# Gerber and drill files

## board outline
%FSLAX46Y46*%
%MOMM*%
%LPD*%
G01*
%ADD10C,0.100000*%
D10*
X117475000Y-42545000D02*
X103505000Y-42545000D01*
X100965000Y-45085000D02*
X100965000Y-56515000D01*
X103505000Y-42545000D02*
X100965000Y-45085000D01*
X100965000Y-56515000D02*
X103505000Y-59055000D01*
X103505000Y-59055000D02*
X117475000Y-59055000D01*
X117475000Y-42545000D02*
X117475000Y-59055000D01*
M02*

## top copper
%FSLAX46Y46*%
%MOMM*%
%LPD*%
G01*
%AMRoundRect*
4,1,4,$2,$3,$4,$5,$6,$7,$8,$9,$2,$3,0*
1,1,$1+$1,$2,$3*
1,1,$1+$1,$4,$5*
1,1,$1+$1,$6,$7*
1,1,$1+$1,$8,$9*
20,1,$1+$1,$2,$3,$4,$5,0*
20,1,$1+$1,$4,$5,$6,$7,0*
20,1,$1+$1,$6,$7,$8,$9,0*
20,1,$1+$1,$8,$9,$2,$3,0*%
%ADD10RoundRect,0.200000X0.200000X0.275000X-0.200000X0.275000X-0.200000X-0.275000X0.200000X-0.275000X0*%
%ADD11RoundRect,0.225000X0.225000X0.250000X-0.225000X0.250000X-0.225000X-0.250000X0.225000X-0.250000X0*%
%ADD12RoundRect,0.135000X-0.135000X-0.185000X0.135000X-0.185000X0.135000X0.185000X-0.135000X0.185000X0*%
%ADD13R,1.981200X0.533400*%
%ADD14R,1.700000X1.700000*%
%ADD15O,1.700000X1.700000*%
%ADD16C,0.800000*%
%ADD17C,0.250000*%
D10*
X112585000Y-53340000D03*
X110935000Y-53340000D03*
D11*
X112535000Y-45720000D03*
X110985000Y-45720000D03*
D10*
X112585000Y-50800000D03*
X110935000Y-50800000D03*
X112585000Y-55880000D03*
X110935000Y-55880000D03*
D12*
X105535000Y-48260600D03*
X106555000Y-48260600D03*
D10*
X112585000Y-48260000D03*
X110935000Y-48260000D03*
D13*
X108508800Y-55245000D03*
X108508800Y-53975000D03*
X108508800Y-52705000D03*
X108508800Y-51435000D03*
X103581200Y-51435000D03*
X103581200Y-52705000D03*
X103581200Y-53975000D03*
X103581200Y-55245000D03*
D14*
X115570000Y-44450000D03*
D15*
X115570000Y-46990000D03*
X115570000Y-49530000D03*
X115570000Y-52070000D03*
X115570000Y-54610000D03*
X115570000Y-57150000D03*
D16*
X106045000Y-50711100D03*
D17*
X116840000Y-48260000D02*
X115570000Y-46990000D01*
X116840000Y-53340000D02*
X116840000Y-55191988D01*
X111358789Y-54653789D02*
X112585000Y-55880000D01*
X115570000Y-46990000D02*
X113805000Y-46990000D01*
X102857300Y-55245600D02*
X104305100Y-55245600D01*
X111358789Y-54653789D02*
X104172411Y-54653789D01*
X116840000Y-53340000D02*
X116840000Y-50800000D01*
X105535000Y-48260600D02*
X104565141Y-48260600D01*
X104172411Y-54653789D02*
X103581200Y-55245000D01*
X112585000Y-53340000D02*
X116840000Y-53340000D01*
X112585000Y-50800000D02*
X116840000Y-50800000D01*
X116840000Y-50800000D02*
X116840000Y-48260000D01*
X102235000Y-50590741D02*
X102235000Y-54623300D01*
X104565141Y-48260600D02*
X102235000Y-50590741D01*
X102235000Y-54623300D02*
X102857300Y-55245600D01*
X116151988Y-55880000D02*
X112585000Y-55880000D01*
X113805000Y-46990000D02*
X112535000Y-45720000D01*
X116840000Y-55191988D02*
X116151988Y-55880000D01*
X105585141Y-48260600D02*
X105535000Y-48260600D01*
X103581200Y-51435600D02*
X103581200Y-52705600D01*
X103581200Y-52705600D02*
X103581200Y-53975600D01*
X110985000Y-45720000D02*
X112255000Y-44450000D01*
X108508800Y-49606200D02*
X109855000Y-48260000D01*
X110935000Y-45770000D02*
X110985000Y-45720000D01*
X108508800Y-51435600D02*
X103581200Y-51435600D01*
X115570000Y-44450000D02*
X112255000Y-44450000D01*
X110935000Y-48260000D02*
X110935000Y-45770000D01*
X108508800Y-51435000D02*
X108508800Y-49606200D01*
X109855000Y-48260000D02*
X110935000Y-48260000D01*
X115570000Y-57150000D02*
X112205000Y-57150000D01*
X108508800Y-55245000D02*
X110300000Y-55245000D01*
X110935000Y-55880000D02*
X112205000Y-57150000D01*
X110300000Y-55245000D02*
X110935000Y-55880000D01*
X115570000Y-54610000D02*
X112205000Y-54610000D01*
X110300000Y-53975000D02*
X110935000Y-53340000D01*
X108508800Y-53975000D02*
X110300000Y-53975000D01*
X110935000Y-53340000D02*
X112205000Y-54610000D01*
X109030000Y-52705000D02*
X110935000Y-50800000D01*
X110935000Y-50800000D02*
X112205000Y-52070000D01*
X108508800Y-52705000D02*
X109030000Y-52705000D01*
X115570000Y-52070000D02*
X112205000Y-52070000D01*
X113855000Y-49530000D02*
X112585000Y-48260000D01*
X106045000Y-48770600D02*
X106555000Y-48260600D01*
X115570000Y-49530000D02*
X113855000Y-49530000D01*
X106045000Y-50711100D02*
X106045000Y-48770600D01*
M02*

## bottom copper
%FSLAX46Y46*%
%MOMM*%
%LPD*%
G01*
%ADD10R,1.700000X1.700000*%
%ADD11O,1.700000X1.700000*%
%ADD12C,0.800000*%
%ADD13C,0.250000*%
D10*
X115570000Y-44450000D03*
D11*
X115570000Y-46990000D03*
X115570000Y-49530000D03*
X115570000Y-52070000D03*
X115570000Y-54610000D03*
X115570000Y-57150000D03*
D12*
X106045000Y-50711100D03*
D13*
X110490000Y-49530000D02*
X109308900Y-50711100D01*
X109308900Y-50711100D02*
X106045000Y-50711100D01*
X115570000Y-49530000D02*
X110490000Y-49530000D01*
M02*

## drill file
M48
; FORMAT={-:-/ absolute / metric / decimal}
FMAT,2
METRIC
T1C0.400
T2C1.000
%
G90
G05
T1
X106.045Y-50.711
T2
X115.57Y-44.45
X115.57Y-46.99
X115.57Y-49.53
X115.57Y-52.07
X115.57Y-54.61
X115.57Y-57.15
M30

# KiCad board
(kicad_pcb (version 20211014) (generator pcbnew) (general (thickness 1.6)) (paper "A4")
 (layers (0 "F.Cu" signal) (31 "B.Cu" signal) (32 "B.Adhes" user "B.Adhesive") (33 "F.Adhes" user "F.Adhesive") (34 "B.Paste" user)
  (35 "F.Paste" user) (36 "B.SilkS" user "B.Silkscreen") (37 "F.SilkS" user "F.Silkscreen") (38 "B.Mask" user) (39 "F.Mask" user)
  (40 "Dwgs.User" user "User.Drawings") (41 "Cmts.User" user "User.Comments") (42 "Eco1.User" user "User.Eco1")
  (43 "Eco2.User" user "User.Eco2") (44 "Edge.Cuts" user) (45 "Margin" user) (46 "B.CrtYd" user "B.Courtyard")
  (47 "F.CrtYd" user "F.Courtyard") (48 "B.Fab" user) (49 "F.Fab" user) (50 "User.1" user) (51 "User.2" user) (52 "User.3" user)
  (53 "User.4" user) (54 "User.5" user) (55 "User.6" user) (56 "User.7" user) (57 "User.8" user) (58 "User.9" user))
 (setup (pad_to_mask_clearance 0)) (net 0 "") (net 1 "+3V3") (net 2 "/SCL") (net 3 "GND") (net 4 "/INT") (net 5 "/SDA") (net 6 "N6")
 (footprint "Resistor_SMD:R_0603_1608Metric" (layer "F.Cu") (at 111.76 53.34 180)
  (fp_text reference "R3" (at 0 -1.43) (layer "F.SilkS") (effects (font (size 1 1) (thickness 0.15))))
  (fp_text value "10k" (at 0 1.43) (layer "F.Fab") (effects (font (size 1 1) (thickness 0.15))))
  (pad "1" smd roundrect (at -0.825 0 180) (size 0.8 0.95) (layers "F.Cu" "F.Paste" "F.Mask") (roundrect_rratio 0.25) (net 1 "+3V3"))
  (pad "2" smd roundrect (at 0.825 0 180) (size 0.8 0.95) (layers "F.Cu" "F.Paste" "F.Mask") (roundrect_rratio 0.25) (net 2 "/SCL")))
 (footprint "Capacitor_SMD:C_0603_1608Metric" (layer "F.Cu") (at 111.76 45.72 180)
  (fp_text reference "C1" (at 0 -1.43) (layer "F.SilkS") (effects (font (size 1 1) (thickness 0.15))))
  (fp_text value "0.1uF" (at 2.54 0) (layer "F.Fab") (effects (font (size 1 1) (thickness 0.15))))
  (pad "1" smd roundrect (at -0.775 0 180) (size 0.9 0.95) (layers "F.Cu" "F.Paste" "F.Mask") (roundrect_rratio 0.25) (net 1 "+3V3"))
  (pad "2" smd roundrect (at 0.775 0 180) (size 0.9 0.95) (layers "F.Cu" "F.Paste" "F.Mask") (roundrect_rratio 0.25) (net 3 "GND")))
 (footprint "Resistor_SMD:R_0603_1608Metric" (layer "F.Cu") (at 111.76 50.8 180)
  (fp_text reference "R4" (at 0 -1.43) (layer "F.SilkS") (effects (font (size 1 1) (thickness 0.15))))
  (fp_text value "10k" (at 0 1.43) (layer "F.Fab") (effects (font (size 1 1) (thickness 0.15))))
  (pad "1" smd roundrect (at -0.825 0 180) (size 0.8 0.95) (layers "F.Cu" "F.Paste" "F.Mask") (roundrect_rratio 0.25) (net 1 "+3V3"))
  (pad "2" smd roundrect (at 0.825 0 180) (size 0.8 0.95) (layers "F.Cu" "F.Paste" "F.Mask") (roundrect_rratio 0.25) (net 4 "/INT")))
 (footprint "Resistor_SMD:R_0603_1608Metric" (layer "F.Cu") (at 111.76 55.88 180)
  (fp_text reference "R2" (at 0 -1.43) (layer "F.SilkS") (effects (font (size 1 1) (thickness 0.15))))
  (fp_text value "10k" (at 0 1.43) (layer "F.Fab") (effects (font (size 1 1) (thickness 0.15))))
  (pad "1" smd roundrect (at -0.825 0 180) (size 0.8 0.95) (layers "F.Cu" "F.Paste" "F.Mask") (roundrect_rratio 0.25) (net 1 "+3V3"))
  (pad "2" smd roundrect (at 0.825 0 180) (size 0.8 0.95) (layers "F.Cu" "F.Paste" "F.Mask") (roundrect_rratio 0.25) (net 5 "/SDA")))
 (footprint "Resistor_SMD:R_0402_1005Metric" (layer "F.Cu") (at 106.045 48.2606)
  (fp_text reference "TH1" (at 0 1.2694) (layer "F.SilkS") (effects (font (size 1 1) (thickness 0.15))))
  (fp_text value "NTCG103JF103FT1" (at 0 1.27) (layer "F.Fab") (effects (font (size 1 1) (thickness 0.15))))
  (pad "1" smd roundrect (at -0.51 0) (size 0.54 0.64) (layers "F.Cu" "F.Paste" "F.Mask") (roundrect_rratio 0.25) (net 1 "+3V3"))
  (pad "2" smd roundrect (at 0.51 0) (size 0.54 0.64) (layers "F.Cu" "F.Paste" "F.Mask") (roundrect_rratio 0.25) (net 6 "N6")))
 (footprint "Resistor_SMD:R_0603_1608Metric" (layer "F.Cu") (at 111.76 48.26 180)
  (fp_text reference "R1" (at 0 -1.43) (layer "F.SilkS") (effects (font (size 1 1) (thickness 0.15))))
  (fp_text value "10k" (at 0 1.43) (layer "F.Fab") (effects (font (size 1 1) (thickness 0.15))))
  (pad "1" smd roundrect (at -0.825 0 180) (size 0.8 0.95) (layers "F.Cu" "F.Paste" "F.Mask") (roundrect_rratio 0.25) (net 6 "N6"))
  (pad "2" smd roundrect (at 0.825 0 180) (size 0.8 0.95) (layers "F.Cu" "F.Paste" "F.Mask") (roundrect_rratio 0.25) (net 3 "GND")))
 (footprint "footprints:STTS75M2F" (layer "F.Cu") (at 106.045 53.34 180)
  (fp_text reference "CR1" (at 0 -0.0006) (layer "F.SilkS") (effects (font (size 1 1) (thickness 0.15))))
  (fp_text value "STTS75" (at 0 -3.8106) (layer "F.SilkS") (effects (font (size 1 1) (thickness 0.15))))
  (pad "1" smd rect locked (at -2.4638 -1.905 180) (size 1.9812 0.5334) (layers "F.Cu" "F.Paste" "F.Mask") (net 5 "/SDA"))
  (pad "2" smd rect locked (at -2.4638 -0.635 180) (size 1.9812 0.5334) (layers "F.Cu" "F.Paste" "F.Mask") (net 2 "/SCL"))
  (pad "3" smd rect locked (at -2.4638 0.635 180) (size 1.9812 0.5334) (layers "F.Cu" "F.Paste" "F.Mask") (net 4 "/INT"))
  (pad "4" smd rect locked (at -2.4638 1.905 180) (size 1.9812 0.5334) (layers "F.Cu" "F.Paste" "F.Mask") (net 3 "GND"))
  (pad "5" smd rect locked (at 2.4638 1.905 180) (size 1.9812 0.5334) (layers "F.Cu" "F.Paste" "F.Mask") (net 3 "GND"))
  (pad "6" smd rect locked (at 2.4638 0.635 180) (size 1.9812 0.5334) (layers "F.Cu" "F.Paste" "F.Mask") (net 3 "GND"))
  (pad "7" smd rect locked (at 2.4638 -0.635 180) (size 1.9812 0.5334) (layers "F.Cu" "F.Paste" "F.Mask") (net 3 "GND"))
  (pad "8" smd rect locked (at 2.4638 -1.905 180) (size 1.9812 0.5334) (layers "F.Cu" "F.Paste" "F.Mask") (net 1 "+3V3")))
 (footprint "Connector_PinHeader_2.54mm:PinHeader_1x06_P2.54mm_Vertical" (layer "F.Cu") (at 115.57 44.45)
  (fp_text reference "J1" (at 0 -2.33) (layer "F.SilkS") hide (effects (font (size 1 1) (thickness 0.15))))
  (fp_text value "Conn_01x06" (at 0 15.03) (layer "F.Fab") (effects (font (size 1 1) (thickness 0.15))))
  (pad "1" thru_hole rect (at 0 0) (size 1.7 1.7) (drill 1) (layers *.Cu *.Mask) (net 3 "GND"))
  (pad "2" thru_hole oval (at 0 2.54) (size 1.7 1.7) (drill 1) (layers *.Cu *.Mask) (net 1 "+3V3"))
  (pad "3" thru_hole oval (at 0 5.08) (size 1.7 1.7) (drill 1) (layers *.Cu *.Mask) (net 6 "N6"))
  (pad "4" thru_hole oval (at 0 7.62) (size 1.7 1.7) (drill 1) (layers *.Cu *.Mask) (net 4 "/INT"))
  (pad "5" thru_hole oval (at 0 10.16) (size 1.7 1.7) (drill 1) (layers *.Cu *.Mask) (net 2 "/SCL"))
  (pad "6" thru_hole oval (at 0 12.7) (size 1.7 1.7) (drill 1) (layers *.Cu *.Mask) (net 5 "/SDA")))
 (gr_line (start 117.475 42.545) (end 103.505 42.545) (layer "Edge.Cuts") (width 0.1))
 (gr_line (start 100.965 45.085) (end 100.965 56.515) (layer "Edge.Cuts") (width 0.1))
 (gr_line (start 103.505 42.545) (end 100.965 45.085) (layer "Edge.Cuts") (width 0.1))
 (gr_line (start 100.965 56.515) (end 103.505 59.055) (layer "Edge.Cuts") (width 0.1))
 (gr_line (start 103.505 59.055) (end 117.475 59.055) (layer "Edge.Cuts") (width 0.1))
 (gr_line (start 117.475 42.545) (end 117.475 59.055) (layer "Edge.Cuts") (width 0.1))
 (segment (start 116.84 48.26) (end 115.57 46.99) (width 0.25) (layer "F.Cu") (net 1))
 (segment (start 116.84 53.34) (end 116.84 55.191988) (width 0.25) (layer "F.Cu") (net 1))
 (segment (start 111.358789 54.653789) (end 112.585 55.88) (width 0.25) (layer "F.Cu") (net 1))
 (segment (start 115.57 46.99) (end 113.805 46.99) (width 0.25) (layer "F.Cu") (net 1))
 (segment (start 102.8573 55.2456) (end 104.3051 55.2456) (width 0.25) (layer "F.Cu") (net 1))
 (segment (start 111.358789 54.653789) (end 104.172411 54.653789) (width 0.25) (layer "F.Cu") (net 1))
 (segment (start 116.84 53.34) (end 116.84 50.8) (width 0.25) (layer "F.Cu") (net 1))
 (segment (start 105.535 48.2606) (end 104.565141 48.2606) (width 0.25) (layer "F.Cu") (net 1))
 (segment (start 104.172411 54.653789) (end 103.5812 55.245) (width 0.25) (layer "F.Cu") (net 1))
 (segment (start 112.585 53.34) (end 116.84 53.34) (width 0.25) (layer "F.Cu") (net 1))
 (segment (start 112.585 50.8) (end 116.84 50.8) (width 0.25) (layer "F.Cu") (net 1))
 (segment (start 116.84 50.8) (end 116.84 48.26) (width 0.25) (layer "F.Cu") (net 1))
 (segment (start 102.235 50.590741) (end 102.235 54.6233) (width 0.25) (layer "F.Cu") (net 1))
 (segment (start 104.565141 48.2606) (end 102.235 50.590741) (width 0.25) (layer "F.Cu") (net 1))
 (segment (start 102.235 54.6233) (end 102.8573 55.2456) (width 0.25) (layer "F.Cu") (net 1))
 (segment (start 116.151988 55.88) (end 112.585 55.88) (width 0.25) (layer "F.Cu") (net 1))
 (segment (start 113.805 46.99) (end 112.535 45.72) (width 0.25) (layer "F.Cu") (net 1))
 (segment (start 116.84 55.191988) (end 116.151988 55.88) (width 0.25) (layer "F.Cu") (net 1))
 (segment (start 105.585141 48.2606) (end 105.535 48.2606) (width 0.25) (layer "F.Cu") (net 1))
 (segment (start 103.5812 51.4356) (end 103.5812 52.7056) (width 0.25) (layer "F.Cu") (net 3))
 (segment (start 103.5812 52.7056) (end 103.5812 53.9756) (width 0.25) (layer "F.Cu") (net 3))
 (segment (start 110.985 45.72) (end 112.255 44.45) (width 0.25) (layer "F.Cu") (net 3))
 (segment (start 108.5088 49.6062) (end 109.855 48.26) (width 0.25) (layer "F.Cu") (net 3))
 (segment (start 110.935 45.77) (end 110.985 45.72) (width 0.25) (layer "F.Cu") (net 3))
 (segment (start 108.5088 51.4356) (end 103.5812 51.4356) (width 0.25) (layer "F.Cu") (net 3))
 (segment (start 115.57 44.45) (end 112.255 44.45) (width 0.25) (layer "F.Cu") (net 3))
 (segment (start 110.935 48.26) (end 110.935 45.77) (width 0.25) (layer "F.Cu") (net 3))
 (segment (start 108.5088 51.435) (end 108.5088 49.6062) (width 0.25) (layer "F.Cu") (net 3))
 (segment (start 109.855 48.26) (end 110.935 48.26) (width 0.25) (layer "F.Cu") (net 3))
 (segment (start 115.57 57.15) (end 112.205 57.15) (width 0.25) (layer "F.Cu") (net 5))
 (segment (start 108.5088 55.245) (end 110.3 55.245) (width 0.25) (layer "F.Cu") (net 5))
 (segment (start 110.935 55.88) (end 112.205 57.15) (width 0.25) (layer "F.Cu") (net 5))
 (segment (start 110.3 55.245) (end 110.935 55.88) (width 0.25) (layer "F.Cu") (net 5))
 (segment (start 115.57 54.61) (end 112.205 54.61) (width 0.25) (layer "F.Cu") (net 2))
 (segment (start 110.3 53.975) (end 110.935 53.34) (width 0.25) (layer "F.Cu") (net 2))
 (segment (start 108.5088 53.975) (end 110.3 53.975) (width 0.25) (layer "F.Cu") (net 2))
 (segment (start 110.935 53.34) (end 112.205 54.61) (width 0.25) (layer "F.Cu") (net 2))
 (segment (start 109.03 52.705) (end 110.935 50.8) (width 0.25) (layer "F.Cu") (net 4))
 (segment (start 110.935 50.8) (end 112.205 52.07) (width 0.25) (layer "F.Cu") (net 4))
 (segment (start 108.5088 52.705) (end 109.03 52.705) (width 0.25) (layer "F.Cu") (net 4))
 (segment (start 115.57 52.07) (end 112.205 52.07) (width 0.25) (layer "F.Cu") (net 4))
 (segment (start 113.855 49.53) (end 112.585 48.26) (width 0.25) (layer "F.Cu") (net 6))
 (segment (start 106.045 48.7706) (end 106.555 48.2606) (width 0.25) (layer "F.Cu") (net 6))
 (segment (start 115.57 49.53) (end 113.855 49.53) (width 0.25) (layer "F.Cu") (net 6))
 (segment (start 106.045 50.7111) (end 106.045 48.7706) (width 0.25) (layer "F.Cu") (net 6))
 (via (at 106.045 50.7111) (size 0.8) (drill 0.4) (layers "F.Cu" "B.Cu") (free) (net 6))
 (segment (start 110.49 49.53) (end 109.3089 50.7111) (width 0.25) (layer "B.Cu") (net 6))
 (segment (start 109.3089 50.7111) (end 106.045 50.7111) (width 0.25) (layer "B.Cu") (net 6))
 (segment (start 115.57 49.53) (end 110.49 49.53) (width 0.25) (layer "B.Cu") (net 6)))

